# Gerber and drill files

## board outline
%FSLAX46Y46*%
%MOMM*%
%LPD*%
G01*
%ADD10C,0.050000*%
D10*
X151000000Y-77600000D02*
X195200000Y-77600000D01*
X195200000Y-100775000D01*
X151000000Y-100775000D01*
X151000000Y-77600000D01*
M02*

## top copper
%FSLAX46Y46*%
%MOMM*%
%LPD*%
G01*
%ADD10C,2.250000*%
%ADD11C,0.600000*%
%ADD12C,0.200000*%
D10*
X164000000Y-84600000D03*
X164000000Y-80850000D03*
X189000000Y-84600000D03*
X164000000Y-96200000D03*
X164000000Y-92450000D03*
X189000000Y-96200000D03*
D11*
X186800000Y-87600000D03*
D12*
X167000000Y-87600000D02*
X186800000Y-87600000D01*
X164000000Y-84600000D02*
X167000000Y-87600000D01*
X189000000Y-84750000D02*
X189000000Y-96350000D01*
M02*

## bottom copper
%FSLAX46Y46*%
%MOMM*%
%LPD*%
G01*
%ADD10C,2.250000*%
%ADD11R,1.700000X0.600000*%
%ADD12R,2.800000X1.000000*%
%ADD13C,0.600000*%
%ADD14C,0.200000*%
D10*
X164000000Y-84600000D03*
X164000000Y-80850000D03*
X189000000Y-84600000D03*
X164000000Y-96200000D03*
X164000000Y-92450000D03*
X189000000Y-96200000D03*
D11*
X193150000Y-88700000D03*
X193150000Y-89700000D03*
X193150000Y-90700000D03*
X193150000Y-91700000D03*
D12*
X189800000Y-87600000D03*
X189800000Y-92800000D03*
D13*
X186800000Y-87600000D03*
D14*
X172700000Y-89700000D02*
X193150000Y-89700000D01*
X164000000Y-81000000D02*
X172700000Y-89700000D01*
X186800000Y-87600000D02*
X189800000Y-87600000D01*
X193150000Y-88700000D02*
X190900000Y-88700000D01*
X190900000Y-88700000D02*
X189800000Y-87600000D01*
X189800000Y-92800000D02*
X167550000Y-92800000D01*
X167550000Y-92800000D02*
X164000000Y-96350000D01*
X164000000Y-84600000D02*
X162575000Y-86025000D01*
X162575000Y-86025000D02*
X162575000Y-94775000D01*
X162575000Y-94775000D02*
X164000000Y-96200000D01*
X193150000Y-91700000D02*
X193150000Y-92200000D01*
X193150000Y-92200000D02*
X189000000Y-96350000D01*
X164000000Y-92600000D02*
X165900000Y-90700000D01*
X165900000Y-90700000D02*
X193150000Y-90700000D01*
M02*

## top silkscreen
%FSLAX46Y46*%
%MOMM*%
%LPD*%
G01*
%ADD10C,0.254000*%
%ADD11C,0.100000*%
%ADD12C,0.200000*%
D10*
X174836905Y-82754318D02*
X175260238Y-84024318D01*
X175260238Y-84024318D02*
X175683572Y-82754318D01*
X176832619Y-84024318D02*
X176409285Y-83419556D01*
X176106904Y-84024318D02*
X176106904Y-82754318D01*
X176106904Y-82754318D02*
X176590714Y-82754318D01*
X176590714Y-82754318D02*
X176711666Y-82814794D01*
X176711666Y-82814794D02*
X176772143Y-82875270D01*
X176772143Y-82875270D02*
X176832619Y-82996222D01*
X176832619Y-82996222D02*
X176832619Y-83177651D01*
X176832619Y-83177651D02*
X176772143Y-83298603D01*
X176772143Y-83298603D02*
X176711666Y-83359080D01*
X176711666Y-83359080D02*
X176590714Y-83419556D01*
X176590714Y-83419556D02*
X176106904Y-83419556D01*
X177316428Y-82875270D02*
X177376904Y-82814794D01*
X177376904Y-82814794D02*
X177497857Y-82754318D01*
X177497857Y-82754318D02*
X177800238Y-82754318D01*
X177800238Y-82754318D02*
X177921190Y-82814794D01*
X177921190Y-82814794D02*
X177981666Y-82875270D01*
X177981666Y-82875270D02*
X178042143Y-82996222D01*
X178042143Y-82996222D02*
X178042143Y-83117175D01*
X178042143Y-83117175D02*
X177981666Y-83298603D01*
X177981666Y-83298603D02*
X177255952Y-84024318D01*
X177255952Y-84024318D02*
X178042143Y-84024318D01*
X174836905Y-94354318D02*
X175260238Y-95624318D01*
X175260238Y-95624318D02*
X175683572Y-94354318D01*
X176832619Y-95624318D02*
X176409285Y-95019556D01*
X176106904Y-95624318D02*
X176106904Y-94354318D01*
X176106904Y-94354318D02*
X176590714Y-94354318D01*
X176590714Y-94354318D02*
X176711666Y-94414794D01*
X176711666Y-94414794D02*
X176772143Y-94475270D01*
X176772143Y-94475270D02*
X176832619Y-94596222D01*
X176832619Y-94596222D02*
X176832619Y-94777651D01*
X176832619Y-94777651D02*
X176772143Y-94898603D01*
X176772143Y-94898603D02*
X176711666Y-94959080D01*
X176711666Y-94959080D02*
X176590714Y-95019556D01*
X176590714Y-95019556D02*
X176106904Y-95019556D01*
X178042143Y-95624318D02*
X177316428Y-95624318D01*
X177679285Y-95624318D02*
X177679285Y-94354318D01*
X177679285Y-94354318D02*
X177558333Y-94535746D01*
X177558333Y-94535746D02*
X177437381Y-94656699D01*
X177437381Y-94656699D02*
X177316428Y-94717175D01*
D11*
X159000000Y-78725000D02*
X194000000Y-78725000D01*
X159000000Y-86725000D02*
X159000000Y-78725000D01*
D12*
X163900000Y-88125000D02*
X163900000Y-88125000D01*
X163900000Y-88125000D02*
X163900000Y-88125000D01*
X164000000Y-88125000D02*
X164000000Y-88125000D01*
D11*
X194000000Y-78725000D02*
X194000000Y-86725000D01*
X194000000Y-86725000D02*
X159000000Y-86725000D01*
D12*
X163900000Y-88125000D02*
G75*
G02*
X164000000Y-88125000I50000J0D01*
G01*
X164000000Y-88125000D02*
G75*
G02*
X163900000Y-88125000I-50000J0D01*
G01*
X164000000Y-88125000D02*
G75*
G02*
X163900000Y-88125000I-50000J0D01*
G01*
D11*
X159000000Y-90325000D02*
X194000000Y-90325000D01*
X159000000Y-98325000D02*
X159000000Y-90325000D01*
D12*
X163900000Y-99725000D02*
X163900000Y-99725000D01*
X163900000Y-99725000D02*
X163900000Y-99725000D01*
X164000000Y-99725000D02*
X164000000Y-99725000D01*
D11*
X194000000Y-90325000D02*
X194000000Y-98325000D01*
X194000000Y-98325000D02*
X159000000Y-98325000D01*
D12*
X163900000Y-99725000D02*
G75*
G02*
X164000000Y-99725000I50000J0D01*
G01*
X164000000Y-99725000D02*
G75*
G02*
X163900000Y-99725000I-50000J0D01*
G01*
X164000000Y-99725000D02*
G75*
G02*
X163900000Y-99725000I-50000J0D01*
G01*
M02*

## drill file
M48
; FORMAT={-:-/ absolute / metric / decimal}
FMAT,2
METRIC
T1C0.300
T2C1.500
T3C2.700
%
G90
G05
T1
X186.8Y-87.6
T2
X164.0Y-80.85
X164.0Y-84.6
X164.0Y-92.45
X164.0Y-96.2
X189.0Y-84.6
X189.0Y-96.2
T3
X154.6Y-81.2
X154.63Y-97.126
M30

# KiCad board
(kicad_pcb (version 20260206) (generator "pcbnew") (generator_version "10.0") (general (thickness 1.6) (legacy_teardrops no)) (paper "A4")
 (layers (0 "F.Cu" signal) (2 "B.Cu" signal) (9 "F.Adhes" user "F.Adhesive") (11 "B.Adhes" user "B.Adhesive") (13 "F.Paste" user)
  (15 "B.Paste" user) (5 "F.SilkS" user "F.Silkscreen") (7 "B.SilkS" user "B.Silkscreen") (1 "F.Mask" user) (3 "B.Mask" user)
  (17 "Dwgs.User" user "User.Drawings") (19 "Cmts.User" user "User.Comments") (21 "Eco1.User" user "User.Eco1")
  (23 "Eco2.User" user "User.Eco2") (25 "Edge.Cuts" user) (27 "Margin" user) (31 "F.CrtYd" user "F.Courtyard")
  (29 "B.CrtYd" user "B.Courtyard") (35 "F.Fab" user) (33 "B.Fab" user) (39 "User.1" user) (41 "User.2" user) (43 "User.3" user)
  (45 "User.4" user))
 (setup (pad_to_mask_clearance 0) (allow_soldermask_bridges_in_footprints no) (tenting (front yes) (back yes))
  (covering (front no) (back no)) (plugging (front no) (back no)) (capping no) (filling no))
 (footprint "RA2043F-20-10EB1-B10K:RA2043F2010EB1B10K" (layer "F.Cu") (at 164 84.6)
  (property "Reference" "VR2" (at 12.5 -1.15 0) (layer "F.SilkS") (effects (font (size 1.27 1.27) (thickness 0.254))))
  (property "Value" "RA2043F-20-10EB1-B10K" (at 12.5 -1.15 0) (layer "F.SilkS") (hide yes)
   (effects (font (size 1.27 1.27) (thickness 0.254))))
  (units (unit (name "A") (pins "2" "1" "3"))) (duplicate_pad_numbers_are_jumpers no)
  (fp_line (start -5 -5.875) (end 30 -5.875) (stroke (width 0.1) (type solid)) (layer "F.SilkS"))
  (fp_line (start -5 2.125) (end -5 -5.875) (stroke (width 0.1) (type solid)) (layer "F.SilkS"))
  (fp_line (start -0.1 3.525) (end -0.1 3.525) (stroke (width 0.2) (type solid)) (layer "F.SilkS"))
  (fp_line (start -0.1 3.525) (end -0.1 3.525) (stroke (width 0.2) (type solid)) (layer "F.SilkS"))
  (fp_line (start 0 3.525) (end 0 3.525) (stroke (width 0.2) (type solid)) (layer "F.SilkS"))
  (fp_line (start 30 -5.875) (end 30 2.125) (stroke (width 0.1) (type solid)) (layer "F.SilkS"))
  (fp_line (start 30 2.125) (end -5 2.125) (stroke (width 0.1) (type solid)) (layer "F.SilkS"))
  (fp_arc (start -0.1 3.525) (mid -0.05 3.475) (end 0 3.525) (stroke (width 0.2) (type solid)) (layer "F.SilkS"))
  (fp_arc (start 0 3.525) (mid -0.05 3.575) (end -0.1 3.525) (stroke (width 0.2) (type solid)) (layer "F.SilkS"))
  (fp_arc (start 0 3.525) (mid -0.05 3.575) (end -0.1 3.525) (stroke (width 0.2) (type solid)) (layer "F.SilkS"))
  (pad "1" thru_hole circle (at 0 0) (size 2.25 2.25) (drill 1.5) (layers "*.Cu" "*.Mask") (remove_unused_layers no) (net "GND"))
  (pad "2" thru_hole circle (at 0 -3.75) (size 2.25 2.25) (drill 1.5) (layers "*.Cu" "*.Mask") (remove_unused_layers no) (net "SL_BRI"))
  (pad "3" thru_hole circle (at 25 0) (size 2.25 2.25) (drill 1.5) (layers "*.Cu" "*.Mask") (remove_unused_layers no) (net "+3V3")))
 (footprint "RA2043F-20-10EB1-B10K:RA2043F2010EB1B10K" (layer "F.Cu") (at 164 96.2)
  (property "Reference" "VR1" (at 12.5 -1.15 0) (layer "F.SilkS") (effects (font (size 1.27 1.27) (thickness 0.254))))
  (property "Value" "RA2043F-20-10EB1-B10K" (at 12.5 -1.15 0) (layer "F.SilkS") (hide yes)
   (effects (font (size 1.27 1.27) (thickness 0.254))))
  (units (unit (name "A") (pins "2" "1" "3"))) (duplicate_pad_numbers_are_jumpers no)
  (fp_line (start -5 -5.875) (end 30 -5.875) (stroke (width 0.1) (type solid)) (layer "F.SilkS"))
  (fp_line (start -5 2.125) (end -5 -5.875) (stroke (width 0.1) (type solid)) (layer "F.SilkS"))
  (fp_line (start -0.1 3.525) (end -0.1 3.525) (stroke (width 0.2) (type solid)) (layer "F.SilkS"))
  (fp_line (start -0.1 3.525) (end -0.1 3.525) (stroke (width 0.2) (type solid)) (layer "F.SilkS"))
  (fp_line (start 0 3.525) (end 0 3.525) (stroke (width 0.2) (type solid)) (layer "F.SilkS"))
  (fp_line (start 30 -5.875) (end 30 2.125) (stroke (width 0.1) (type solid)) (layer "F.SilkS"))
  (fp_line (start 30 2.125) (end -5 2.125) (stroke (width 0.1) (type solid)) (layer "F.SilkS"))
  (fp_arc (start -0.1 3.525) (mid -0.05 3.475) (end 0 3.525) (stroke (width 0.2) (type solid)) (layer "F.SilkS"))
  (fp_arc (start 0 3.525) (mid -0.05 3.575) (end -0.1 3.525) (stroke (width 0.2) (type solid)) (layer "F.SilkS"))
  (fp_arc (start 0 3.525) (mid -0.05 3.575) (end -0.1 3.525) (stroke (width 0.2) (type solid)) (layer "F.SilkS"))
  (pad "1" thru_hole circle (at 0 0) (size 2.25 2.25) (drill 1.5) (layers "*.Cu" "*.Mask") (remove_unused_layers no) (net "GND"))
  (pad "2" thru_hole circle (at 0 -3.75) (size 2.25 2.25) (drill 1.5) (layers "*.Cu" "*.Mask") (remove_unused_layers no) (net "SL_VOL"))
  (pad "3" thru_hole circle (at 25 0) (size 2.25 2.25) (drill 1.5) (layers "*.Cu" "*.Mask") (remove_unused_layers no) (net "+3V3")))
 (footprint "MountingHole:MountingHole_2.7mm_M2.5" (layer "B.Cu") (at 154.6 81.2 -90)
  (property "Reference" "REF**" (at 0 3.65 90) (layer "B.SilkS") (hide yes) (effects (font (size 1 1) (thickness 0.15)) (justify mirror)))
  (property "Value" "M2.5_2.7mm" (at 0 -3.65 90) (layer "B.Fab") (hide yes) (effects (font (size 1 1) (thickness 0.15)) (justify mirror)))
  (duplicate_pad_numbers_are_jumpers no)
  (pad "" np_thru_hole circle (at 0 0 270) (size 2.7 2.7) (drill 2.7) (layers "*.Cu" "*.Mask")))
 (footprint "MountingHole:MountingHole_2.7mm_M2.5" (layer "B.Cu") (at 154.62966 97.125849 -90)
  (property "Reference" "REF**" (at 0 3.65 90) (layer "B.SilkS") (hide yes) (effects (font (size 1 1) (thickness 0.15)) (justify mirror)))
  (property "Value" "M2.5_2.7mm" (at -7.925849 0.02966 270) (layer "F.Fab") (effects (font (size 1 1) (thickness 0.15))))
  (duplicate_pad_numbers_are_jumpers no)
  (pad "" np_thru_hole circle (at 0 0 270) (size 2.7 2.7) (drill 2.7) (layers "*.Cu" "*.Mask")))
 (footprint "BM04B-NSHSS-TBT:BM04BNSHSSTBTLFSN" (layer "B.Cu") (at 190.925 90.2 90)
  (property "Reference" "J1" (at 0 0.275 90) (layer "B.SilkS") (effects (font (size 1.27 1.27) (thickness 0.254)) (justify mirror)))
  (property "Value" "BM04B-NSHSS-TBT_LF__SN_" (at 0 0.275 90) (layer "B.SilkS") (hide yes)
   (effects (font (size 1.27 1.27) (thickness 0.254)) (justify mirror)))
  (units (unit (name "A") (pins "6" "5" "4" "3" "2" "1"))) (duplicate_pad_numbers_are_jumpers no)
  (pad "1" smd rect (at 1.5 2.225 90) (size 0.6 1.7) (layers "B.Cu" "B.Mask" "B.Paste") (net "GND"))
  (pad "2" smd rect (at 0.5 2.225 90) (size 0.6 1.7) (layers "B.Cu" "B.Mask" "B.Paste") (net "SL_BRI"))
  (pad "3" smd rect (at -0.5 2.225 90) (size 0.6 1.7) (layers "B.Cu" "B.Mask" "B.Paste") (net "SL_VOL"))
  (pad "4" smd rect (at -1.5 2.225 90) (size 0.6 1.7) (layers "B.Cu" "B.Mask" "B.Paste") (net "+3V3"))
  (pad "5" smd rect (at 2.6 -1.125 90) (size 1 2.8) (layers "B.Cu" "B.Mask" "B.Paste") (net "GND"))
  (pad "6" smd rect (at -2.6 -1.125 90) (size 1 2.8) (layers "B.Cu" "B.Mask" "B.Paste") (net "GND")))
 (gr_rect (start 151 77.6) (end 195.2 100.775) (stroke (width 0.05) (type solid)) (fill no) (layer "Edge.Cuts"))
 (segment (start 172.7 89.7) (end 193.15 89.7) (width 0.2) (layer "B.Cu") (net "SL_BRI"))
 (segment (start 164 81) (end 172.7 89.7) (width 0.2) (layer "B.Cu") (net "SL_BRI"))
 (segment (start 167 87.6) (end 186.8 87.6) (width 0.2) (layer "F.Cu") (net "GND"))
 (segment (start 164 84.6) (end 167 87.6) (width 0.2) (layer "F.Cu") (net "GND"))
 (via (at 186.8 87.6) (size 0.6) (drill 0.3) (layers "F.Cu" "B.Cu") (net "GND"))
 (segment (start 186.8 87.6) (end 189.8 87.6) (width 0.2) (layer "B.Cu") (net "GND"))
 (segment (start 193.15 88.7) (end 190.9 88.7) (width 0.2) (layer "B.Cu") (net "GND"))
 (segment (start 190.9 88.7) (end 189.8 87.6) (width 0.2) (layer "B.Cu") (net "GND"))
 (segment (start 189.8 92.8) (end 167.55 92.8) (width 0.2) (layer "B.Cu") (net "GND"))
 (segment (start 167.55 92.8) (end 164 96.35) (width 0.2) (layer "B.Cu") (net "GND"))
 (segment (start 164 84.6) (end 162.575 86.025) (width 0.2) (layer "B.Cu") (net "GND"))
 (segment (start 162.575 86.025) (end 162.575 94.775) (width 0.2) (layer "B.Cu") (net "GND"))
 (segment (start 162.575 94.775) (end 164 96.2) (width 0.2) (layer "B.Cu") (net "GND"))
 (segment (start 189 84.75) (end 189 96.35) (width 0.2) (layer "F.Cu") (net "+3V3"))
 (segment (start 193.15 91.7) (end 193.15 92.2) (width 0.2) (layer "B.Cu") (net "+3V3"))
 (segment (start 193.15 92.2) (end 189 96.35) (width 0.2) (layer "B.Cu") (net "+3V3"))
 (segment (start 164 92.6) (end 165.9 90.7) (width 0.2) (layer "B.Cu") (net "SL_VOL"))
 (segment (start 165.9 90.7) (end 193.15 90.7) (width 0.2) (layer "B.Cu") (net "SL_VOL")))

